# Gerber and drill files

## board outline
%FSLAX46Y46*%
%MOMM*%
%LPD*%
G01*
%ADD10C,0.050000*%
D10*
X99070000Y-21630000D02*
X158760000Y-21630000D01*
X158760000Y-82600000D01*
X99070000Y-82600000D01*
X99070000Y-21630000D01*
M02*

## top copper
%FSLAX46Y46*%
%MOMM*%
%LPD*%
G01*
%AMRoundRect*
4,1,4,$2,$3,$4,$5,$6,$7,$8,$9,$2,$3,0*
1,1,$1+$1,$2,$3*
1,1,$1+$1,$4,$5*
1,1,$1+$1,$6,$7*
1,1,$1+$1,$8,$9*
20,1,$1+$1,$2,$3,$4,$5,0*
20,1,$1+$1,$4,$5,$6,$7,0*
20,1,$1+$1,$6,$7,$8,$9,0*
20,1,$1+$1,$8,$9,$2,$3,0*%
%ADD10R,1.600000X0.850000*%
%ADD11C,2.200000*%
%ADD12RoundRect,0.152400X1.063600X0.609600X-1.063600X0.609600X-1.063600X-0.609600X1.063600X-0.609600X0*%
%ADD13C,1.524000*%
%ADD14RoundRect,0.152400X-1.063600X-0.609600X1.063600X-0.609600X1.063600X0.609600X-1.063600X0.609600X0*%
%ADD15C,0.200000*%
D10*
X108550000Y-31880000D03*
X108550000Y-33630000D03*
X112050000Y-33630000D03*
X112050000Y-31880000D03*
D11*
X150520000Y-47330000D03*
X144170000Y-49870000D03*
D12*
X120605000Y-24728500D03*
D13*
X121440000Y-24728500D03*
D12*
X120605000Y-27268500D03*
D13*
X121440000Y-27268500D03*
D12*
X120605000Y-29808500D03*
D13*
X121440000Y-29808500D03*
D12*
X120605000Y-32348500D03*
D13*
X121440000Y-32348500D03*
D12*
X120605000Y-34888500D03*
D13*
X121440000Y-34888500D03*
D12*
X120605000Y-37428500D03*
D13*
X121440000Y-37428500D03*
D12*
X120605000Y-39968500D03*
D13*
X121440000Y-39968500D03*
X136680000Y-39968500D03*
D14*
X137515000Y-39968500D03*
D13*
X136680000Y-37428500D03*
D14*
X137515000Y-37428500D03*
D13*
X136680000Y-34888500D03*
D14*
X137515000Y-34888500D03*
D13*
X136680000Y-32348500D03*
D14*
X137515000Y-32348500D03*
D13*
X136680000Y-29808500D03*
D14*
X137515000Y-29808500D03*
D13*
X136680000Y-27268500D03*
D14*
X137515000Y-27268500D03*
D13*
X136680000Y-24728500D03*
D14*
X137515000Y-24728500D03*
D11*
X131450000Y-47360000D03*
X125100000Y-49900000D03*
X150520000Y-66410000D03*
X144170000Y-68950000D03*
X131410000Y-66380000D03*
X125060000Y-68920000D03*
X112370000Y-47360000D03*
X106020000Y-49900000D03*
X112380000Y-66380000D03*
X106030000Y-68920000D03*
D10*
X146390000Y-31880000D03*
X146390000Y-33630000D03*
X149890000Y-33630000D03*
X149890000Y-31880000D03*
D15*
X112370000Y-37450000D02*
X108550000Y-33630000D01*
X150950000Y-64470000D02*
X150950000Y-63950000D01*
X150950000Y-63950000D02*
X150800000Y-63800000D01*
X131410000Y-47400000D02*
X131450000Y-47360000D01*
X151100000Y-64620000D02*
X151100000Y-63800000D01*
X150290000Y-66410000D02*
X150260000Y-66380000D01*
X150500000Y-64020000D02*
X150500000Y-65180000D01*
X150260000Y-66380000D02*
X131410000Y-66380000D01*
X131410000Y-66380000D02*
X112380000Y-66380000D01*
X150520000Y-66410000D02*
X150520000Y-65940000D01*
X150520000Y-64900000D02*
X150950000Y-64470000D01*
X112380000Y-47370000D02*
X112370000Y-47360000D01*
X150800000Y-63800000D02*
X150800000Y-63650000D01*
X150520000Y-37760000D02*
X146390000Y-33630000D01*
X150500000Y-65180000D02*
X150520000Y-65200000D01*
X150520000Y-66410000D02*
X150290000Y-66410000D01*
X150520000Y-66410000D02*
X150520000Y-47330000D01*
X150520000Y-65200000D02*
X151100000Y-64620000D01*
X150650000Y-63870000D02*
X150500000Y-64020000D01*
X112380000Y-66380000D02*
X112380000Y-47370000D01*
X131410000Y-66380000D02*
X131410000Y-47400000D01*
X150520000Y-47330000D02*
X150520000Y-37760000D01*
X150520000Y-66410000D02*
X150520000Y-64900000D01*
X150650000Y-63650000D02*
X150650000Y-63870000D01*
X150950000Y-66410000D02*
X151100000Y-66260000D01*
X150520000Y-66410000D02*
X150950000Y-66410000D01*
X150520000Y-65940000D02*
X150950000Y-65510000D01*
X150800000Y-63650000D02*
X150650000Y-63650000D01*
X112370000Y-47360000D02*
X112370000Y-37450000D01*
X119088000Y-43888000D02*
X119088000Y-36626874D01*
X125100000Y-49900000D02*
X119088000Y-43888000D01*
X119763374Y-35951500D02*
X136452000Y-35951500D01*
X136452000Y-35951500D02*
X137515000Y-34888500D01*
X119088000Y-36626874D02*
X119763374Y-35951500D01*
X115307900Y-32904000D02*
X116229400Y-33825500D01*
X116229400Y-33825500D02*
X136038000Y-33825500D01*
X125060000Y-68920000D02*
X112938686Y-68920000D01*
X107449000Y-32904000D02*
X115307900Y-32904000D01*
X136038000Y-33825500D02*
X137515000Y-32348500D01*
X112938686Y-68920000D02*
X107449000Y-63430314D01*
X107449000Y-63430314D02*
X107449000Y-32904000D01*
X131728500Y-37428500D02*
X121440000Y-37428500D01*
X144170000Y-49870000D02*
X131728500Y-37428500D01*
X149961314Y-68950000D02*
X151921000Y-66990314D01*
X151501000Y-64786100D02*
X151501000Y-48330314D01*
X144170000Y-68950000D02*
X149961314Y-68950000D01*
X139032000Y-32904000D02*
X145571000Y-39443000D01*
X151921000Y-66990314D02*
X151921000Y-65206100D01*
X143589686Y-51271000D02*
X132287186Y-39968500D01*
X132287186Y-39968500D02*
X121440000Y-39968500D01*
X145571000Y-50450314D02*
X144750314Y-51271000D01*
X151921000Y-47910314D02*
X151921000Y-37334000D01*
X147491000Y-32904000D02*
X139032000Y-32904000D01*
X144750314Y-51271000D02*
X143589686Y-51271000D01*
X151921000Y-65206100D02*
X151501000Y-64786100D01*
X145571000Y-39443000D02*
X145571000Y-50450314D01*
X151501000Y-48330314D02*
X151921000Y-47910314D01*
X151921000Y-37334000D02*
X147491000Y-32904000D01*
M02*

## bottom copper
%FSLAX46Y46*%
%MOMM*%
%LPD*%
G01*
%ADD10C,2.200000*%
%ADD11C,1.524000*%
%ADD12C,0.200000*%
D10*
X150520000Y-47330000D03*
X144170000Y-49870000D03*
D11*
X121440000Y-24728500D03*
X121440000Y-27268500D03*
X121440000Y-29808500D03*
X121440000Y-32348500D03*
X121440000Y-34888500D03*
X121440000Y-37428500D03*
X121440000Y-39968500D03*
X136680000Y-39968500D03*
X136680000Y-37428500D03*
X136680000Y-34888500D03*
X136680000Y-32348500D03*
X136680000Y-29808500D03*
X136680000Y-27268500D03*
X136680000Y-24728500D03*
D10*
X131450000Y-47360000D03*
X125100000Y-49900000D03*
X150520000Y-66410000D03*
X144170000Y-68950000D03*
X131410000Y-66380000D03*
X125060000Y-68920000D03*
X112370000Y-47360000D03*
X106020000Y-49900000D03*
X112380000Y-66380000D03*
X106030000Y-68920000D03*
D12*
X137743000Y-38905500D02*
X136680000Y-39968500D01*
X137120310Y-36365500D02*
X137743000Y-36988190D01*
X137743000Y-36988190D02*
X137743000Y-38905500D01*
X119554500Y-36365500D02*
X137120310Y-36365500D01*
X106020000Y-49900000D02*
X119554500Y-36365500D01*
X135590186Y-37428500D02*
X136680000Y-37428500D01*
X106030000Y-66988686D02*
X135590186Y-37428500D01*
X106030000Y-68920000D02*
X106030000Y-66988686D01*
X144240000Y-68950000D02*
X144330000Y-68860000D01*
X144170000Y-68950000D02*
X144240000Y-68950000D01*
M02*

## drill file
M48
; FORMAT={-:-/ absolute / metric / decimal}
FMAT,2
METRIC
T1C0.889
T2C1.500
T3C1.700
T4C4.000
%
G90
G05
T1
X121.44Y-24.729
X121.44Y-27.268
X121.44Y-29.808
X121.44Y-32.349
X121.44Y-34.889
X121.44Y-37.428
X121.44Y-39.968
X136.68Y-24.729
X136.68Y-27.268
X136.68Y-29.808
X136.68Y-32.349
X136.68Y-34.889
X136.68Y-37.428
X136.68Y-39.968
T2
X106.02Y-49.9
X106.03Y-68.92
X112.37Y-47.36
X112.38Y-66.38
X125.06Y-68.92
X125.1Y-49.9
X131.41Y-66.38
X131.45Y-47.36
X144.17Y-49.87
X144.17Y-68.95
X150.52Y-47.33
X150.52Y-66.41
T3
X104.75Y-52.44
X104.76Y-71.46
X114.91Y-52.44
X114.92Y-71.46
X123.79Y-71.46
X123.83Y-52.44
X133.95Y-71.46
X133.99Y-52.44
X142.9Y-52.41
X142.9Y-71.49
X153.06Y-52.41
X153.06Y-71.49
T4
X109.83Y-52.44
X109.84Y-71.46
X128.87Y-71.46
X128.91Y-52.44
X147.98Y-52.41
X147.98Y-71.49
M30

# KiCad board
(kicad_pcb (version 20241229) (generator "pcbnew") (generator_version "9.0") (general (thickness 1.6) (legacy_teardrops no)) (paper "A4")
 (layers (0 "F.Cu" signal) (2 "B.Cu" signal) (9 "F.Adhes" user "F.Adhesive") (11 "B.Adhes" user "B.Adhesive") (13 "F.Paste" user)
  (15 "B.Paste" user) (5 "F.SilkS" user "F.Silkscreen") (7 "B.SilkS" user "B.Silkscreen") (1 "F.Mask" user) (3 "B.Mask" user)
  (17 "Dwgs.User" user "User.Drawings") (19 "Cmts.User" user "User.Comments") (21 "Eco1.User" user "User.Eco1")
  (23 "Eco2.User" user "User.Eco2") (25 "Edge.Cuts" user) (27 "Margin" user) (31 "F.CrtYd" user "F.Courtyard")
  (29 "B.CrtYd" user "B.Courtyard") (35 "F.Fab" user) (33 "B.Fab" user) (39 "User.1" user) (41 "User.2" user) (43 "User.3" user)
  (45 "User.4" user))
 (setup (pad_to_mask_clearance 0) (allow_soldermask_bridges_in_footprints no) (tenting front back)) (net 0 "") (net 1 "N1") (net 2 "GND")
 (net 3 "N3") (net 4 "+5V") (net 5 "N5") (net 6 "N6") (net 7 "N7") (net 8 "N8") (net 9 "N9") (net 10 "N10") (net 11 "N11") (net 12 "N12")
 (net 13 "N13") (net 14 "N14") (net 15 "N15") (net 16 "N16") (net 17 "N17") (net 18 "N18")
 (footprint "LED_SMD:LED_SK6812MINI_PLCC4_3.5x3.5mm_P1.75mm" (layer "F.Cu") (at 110.3 32.755)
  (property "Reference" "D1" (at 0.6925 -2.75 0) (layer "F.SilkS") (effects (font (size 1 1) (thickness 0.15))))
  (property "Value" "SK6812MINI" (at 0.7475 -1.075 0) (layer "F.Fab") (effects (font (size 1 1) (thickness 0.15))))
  (pad "1" smd rect (at -1.75 -0.875) (size 1.6 0.85) (layers "F.Cu" "F.Mask" "F.Paste") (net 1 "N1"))
  (pad "2" smd rect (at -1.75 0.875) (size 1.6 0.85) (layers "F.Cu" "F.Mask" "F.Paste") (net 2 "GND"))
  (pad "3" smd rect (at 1.75 0.875) (size 1.6 0.85) (layers "F.Cu" "F.Mask" "F.Paste") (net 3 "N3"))
  (pad "4" smd rect (at 1.75 -0.875) (size 1.6 0.85) (layers "F.Cu" "F.Mask" "F.Paste") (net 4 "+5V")))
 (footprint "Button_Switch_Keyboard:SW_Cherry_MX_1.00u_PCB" (layer "F.Cu") (at 150.52 47.33)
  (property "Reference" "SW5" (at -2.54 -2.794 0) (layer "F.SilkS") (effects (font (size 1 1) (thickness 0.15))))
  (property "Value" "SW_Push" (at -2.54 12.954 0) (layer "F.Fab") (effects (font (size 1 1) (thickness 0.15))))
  (pad "" np_thru_hole circle (at -7.62 5.08) (size 1.7 1.7) (drill 1.7) (layers "*.Cu" "*.Mask"))
  (pad "" np_thru_hole circle (at -2.54 5.08) (size 4 4) (drill 4) (layers "*.Cu" "*.Mask"))
  (pad "" np_thru_hole circle (at 2.54 5.08) (size 1.7 1.7) (drill 1.7) (layers "*.Cu" "*.Mask"))
  (pad "1" thru_hole circle (at 0 0) (size 2.2 2.2) (drill 1.5) (layers "*.Cu" "*.Mask") (remove_unused_layers no) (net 2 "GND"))
  (pad "2" thru_hole circle (at -6.35 2.54) (size 2.2 2.2) (drill 1.5) (layers "*.Cu" "*.Mask") (remove_unused_layers no) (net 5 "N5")))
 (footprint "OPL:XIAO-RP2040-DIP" (layer "F.Cu") (at 129.06 32.3485)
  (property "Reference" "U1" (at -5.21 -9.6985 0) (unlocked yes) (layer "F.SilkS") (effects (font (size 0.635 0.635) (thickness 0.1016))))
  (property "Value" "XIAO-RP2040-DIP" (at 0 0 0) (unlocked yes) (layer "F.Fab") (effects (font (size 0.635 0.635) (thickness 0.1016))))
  (pad "1" smd roundrect (at -8.455 -7.62 180) (size 2.432 1.524) (layers "F.Cu" "F.Mask") (roundrect_rratio 0.1) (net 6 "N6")
   (thermal_bridge_angle 45))
  (pad "1" thru_hole circle (at -7.62 -7.62 180) (size 1.524 1.524) (drill 0.889) (layers "*.Cu" "*.Mask") (remove_unused_layers no)
   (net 6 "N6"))
  (pad "2" smd roundrect (at -8.455 -5.08 180) (size 2.432 1.524) (layers "F.Cu" "F.Mask") (roundrect_rratio 0.1) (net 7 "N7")
   (thermal_bridge_angle 45))
  (pad "2" thru_hole circle (at -7.62 -5.08 180) (size 1.524 1.524) (drill 0.889) (layers "*.Cu" "*.Mask") (remove_unused_layers no)
   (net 7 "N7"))
  (pad "3" smd roundrect (at -8.455 -2.54 180) (size 2.432 1.524) (layers "F.Cu" "F.Mask") (roundrect_rratio 0.1) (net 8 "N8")
   (thermal_bridge_angle 45))
  (pad "3" thru_hole circle (at -7.62 -2.54 180) (size 1.524 1.524) (drill 0.889) (layers "*.Cu" "*.Mask") (remove_unused_layers no)
   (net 8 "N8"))
  (pad "4" smd roundrect (at -8.455 0 180) (size 2.432 1.524) (layers "F.Cu" "F.Mask") (roundrect_rratio 0.1) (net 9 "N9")
   (thermal_bridge_angle 45))
  (pad "4" thru_hole circle (at -7.62 0 180) (size 1.524 1.524) (drill 0.889) (layers "*.Cu" "*.Mask") (remove_unused_layers no)
   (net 9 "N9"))
  (pad "5" smd roundrect (at -8.455 2.54 180) (size 2.432 1.524) (layers "F.Cu" "F.Mask") (roundrect_rratio 0.1) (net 3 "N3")
   (thermal_bridge_angle 45))
  (pad "5" thru_hole circle (at -7.62 2.54 180) (size 1.524 1.524) (drill 0.889) (layers "*.Cu" "*.Mask") (remove_unused_layers no)
   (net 3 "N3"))
  (pad "6" smd roundrect (at -8.455 5.08 180) (size 2.432 1.524) (layers "F.Cu" "F.Mask") (roundrect_rratio 0.1) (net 5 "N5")
   (thermal_bridge_angle 45))
  (pad "6" thru_hole circle (at -7.62 5.08 180) (size 1.524 1.524) (drill 0.889) (layers "*.Cu" "*.Mask") (remove_unused_layers no)
   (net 5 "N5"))
  (pad "7" smd roundrect (at -8.455 7.62 180) (size 2.432 1.524) (layers "F.Cu" "F.Mask") (roundrect_rratio 0.1) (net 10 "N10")
   (thermal_bridge_angle 45))
  (pad "7" thru_hole circle (at -7.62 7.62 180) (size 1.524 1.524) (drill 0.889) (layers "*.Cu" "*.Mask") (remove_unused_layers no)
   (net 10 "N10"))
  (pad "8" thru_hole circle (at 7.62 7.62) (size 1.524 1.524) (drill 0.889) (layers "*.Cu" "*.Mask") (remove_unused_layers no)
   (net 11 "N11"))
  (pad "8" smd roundrect (at 8.455 7.62) (size 2.432 1.524) (layers "F.Cu" "F.Mask") (roundrect_rratio 0.1) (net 11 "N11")
   (thermal_bridge_angle 45))
  (pad "9" thru_hole circle (at 7.62 5.08) (size 1.524 1.524) (drill 0.889) (layers "*.Cu" "*.Mask") (remove_unused_layers no)
   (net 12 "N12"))
  (pad "9" smd roundrect (at 8.455 5.08) (size 2.432 1.524) (layers "F.Cu" "F.Mask") (roundrect_rratio 0.1) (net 12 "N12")
   (thermal_bridge_angle 45))
  (pad "10" thru_hole circle (at 7.62 2.54) (size 1.524 1.524) (drill 0.889) (layers "*.Cu" "*.Mask") (remove_unused_layers no)
   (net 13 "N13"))
  (pad "10" smd roundrect (at 8.455 2.54) (size 2.432 1.524) (layers "F.Cu" "F.Mask") (roundrect_rratio 0.1) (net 13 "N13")
   (thermal_bridge_angle 45))
  (pad "11" thru_hole circle (at 7.62 0) (size 1.524 1.524) (drill 0.889) (layers "*.Cu" "*.Mask") (remove_unused_layers no) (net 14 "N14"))
  (pad "11" smd roundrect (at 8.455 0) (size 2.432 1.524) (layers "F.Cu" "F.Mask") (roundrect_rratio 0.1) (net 14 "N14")
   (thermal_bridge_angle 45))
  (pad "12" thru_hole circle (at 7.62 -2.54) (size 1.524 1.524) (drill 0.889) (layers "*.Cu" "*.Mask") (remove_unused_layers no)
   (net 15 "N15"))
  (pad "12" smd roundrect (at 8.455 -2.54) (size 2.432 1.524) (layers "F.Cu" "F.Mask") (roundrect_rratio 0.1) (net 15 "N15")
   (thermal_bridge_angle 45))
  (pad "13" thru_hole circle (at 7.62 -5.08) (size 1.524 1.524) (drill 0.889) (layers "*.Cu" "*.Mask") (remove_unused_layers no)
   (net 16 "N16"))
  (pad "13" smd roundrect (at 8.455 -5.08) (size 2.432 1.524) (layers "F.Cu" "F.Mask") (roundrect_rratio 0.1) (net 16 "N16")
   (thermal_bridge_angle 45))
  (pad "14" thru_hole circle (at 7.62 -7.62) (size 1.524 1.524) (drill 0.889) (layers "*.Cu" "*.Mask") (remove_unused_layers no)
   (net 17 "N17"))
  (pad "14" smd roundrect (at 8.455 -7.62) (size 2.432 1.524) (layers "F.Cu" "F.Mask") (roundrect_rratio 0.1) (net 17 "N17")
   (thermal_bridge_angle 45)))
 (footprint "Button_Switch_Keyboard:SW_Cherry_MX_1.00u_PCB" (layer "F.Cu") (at 131.45 47.36)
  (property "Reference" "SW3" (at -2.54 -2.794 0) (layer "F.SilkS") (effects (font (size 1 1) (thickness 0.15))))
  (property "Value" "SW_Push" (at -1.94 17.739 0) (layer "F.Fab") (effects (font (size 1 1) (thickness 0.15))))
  (pad "" np_thru_hole circle (at -7.62 5.08) (size 1.7 1.7) (drill 1.7) (layers "*.Cu" "*.Mask"))
  (pad "" np_thru_hole circle (at -2.54 5.08) (size 4 4) (drill 4) (layers "*.Cu" "*.Mask"))
  (pad "" np_thru_hole circle (at 2.54 5.08) (size 1.7 1.7) (drill 1.7) (layers "*.Cu" "*.Mask"))
  (pad "1" thru_hole circle (at 0 0) (size 2.2 2.2) (drill 1.5) (layers "*.Cu" "*.Mask") (remove_unused_layers no) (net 2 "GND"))
  (pad "2" thru_hole circle (at -6.35 2.54) (size 2.2 2.2) (drill 1.5) (layers "*.Cu" "*.Mask") (remove_unused_layers no) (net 13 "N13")))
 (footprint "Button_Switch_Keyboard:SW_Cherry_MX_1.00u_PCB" (layer "F.Cu") (at 150.52 66.41)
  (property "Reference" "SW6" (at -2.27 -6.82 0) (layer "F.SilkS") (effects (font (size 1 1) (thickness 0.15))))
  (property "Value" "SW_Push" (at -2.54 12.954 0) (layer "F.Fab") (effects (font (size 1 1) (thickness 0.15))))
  (pad "" np_thru_hole circle (at -7.62 5.08) (size 1.7 1.7) (drill 1.7) (layers "*.Cu" "*.Mask"))
  (pad "" np_thru_hole circle (at -2.54 5.08) (size 4 4) (drill 4) (layers "*.Cu" "*.Mask"))
  (pad "" np_thru_hole circle (at 2.54 5.08) (size 1.7 1.7) (drill 1.7) (layers "*.Cu" "*.Mask"))
  (pad "1" thru_hole circle (at 0 0) (size 2.2 2.2) (drill 1.5) (layers "*.Cu" "*.Mask") (remove_unused_layers no) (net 2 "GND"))
  (pad "2" thru_hole circle (at -6.35 2.54) (size 2.2 2.2) (drill 1.5) (layers "*.Cu" "*.Mask") (remove_unused_layers no) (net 10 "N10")))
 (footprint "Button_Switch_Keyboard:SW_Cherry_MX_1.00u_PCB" (layer "F.Cu") (at 131.41 66.38)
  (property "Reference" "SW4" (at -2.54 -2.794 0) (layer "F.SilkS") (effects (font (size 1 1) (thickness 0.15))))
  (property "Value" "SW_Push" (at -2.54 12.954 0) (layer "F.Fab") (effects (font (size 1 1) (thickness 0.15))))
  (pad "" np_thru_hole circle (at -7.62 5.08) (size 1.7 1.7) (drill 1.7) (layers "*.Cu" "*.Mask"))
  (pad "" np_thru_hole circle (at -2.54 5.08) (size 4 4) (drill 4) (layers "*.Cu" "*.Mask"))
  (pad "" np_thru_hole circle (at 2.54 5.08) (size 1.7 1.7) (drill 1.7) (layers "*.Cu" "*.Mask"))
  (pad "1" thru_hole circle (at 0 0) (size 2.2 2.2) (drill 1.5) (layers "*.Cu" "*.Mask") (remove_unused_layers no) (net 2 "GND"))
  (pad "2" thru_hole circle (at -6.35 2.54) (size 2.2 2.2) (drill 1.5) (layers "*.Cu" "*.Mask") (remove_unused_layers no) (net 14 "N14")))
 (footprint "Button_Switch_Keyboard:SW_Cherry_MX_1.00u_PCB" (layer "F.Cu") (at 112.37 47.36)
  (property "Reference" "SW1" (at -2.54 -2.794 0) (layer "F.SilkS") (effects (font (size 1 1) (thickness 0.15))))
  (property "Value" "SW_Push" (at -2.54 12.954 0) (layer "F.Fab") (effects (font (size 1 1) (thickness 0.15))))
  (pad "" np_thru_hole circle (at -7.62 5.08) (size 1.7 1.7) (drill 1.7) (layers "*.Cu" "*.Mask"))
  (pad "" np_thru_hole circle (at -2.54 5.08) (size 4 4) (drill 4) (layers "*.Cu" "*.Mask"))
  (pad "" np_thru_hole circle (at 2.54 5.08) (size 1.7 1.7) (drill 1.7) (layers "*.Cu" "*.Mask"))
  (pad "1" thru_hole circle (at 0 0) (size 2.2 2.2) (drill 1.5) (layers "*.Cu" "*.Mask") (remove_unused_layers no) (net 2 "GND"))
  (pad "2" thru_hole circle (at -6.35 2.54) (size 2.2 2.2) (drill 1.5) (layers "*.Cu" "*.Mask") (remove_unused_layers no) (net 11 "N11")))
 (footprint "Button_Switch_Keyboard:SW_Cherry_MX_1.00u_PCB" (layer "F.Cu") (at 112.38 66.38)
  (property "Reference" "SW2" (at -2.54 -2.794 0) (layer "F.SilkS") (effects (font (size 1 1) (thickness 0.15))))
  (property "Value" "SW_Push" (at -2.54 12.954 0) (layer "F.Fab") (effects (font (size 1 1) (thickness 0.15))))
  (pad "" np_thru_hole circle (at -7.62 5.08) (size 1.7 1.7) (drill 1.7) (layers "*.Cu" "*.Mask"))
  (pad "" np_thru_hole circle (at -2.54 5.08) (size 4 4) (drill 4) (layers "*.Cu" "*.Mask"))
  (pad "" np_thru_hole circle (at 2.54 5.08) (size 1.7 1.7) (drill 1.7) (layers "*.Cu" "*.Mask"))
  (pad "1" thru_hole circle (at 0 0) (size 2.2 2.2) (drill 1.5) (layers "*.Cu" "*.Mask") (remove_unused_layers no) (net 2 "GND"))
  (pad "2" thru_hole circle (at -6.35 2.54) (size 2.2 2.2) (drill 1.5) (layers "*.Cu" "*.Mask") (remove_unused_layers no) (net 12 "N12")))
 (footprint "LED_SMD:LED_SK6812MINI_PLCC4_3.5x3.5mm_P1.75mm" (layer "F.Cu") (at 148.14 32.755)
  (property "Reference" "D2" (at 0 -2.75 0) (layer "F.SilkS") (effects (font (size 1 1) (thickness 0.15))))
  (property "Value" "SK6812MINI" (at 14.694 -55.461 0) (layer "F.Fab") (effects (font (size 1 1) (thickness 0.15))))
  (pad "1" smd rect (at -1.75 -0.875) (size 1.6 0.85) (layers "F.Cu" "F.Mask" "F.Paste") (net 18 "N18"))
  (pad "2" smd rect (at -1.75 0.875) (size 1.6 0.85) (layers "F.Cu" "F.Mask" "F.Paste") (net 2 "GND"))
  (pad "3" smd rect (at 1.75 0.875) (size 1.6 0.85) (layers "F.Cu" "F.Mask" "F.Paste") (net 1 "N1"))
  (pad "4" smd rect (at 1.75 -0.875) (size 1.6 0.85) (layers "F.Cu" "F.Mask" "F.Paste") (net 4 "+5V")))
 (gr_rect (start 99.07 21.63) (end 158.76 82.6) (stroke (width 0.05) (type default)) (fill no) (layer "Edge.Cuts"))
 (segment (start 112.37 37.45) (end 108.55 33.63) (width 0.2) (layer "F.Cu") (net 2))
 (segment (start 150.95 64.47) (end 150.95 63.95) (width 0.2) (layer "F.Cu") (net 2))
 (segment (start 150.95 63.95) (end 150.8 63.8) (width 0.2) (layer "F.Cu") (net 2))
 (segment (start 131.41 47.4) (end 131.45 47.36) (width 0.2) (layer "F.Cu") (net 2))
 (segment (start 151.1 64.62) (end 151.1 63.8) (width 0.2) (layer "F.Cu") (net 2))
 (segment (start 150.29 66.41) (end 150.26 66.38) (width 0.2) (layer "F.Cu") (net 2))
 (segment (start 150.5 64.02) (end 150.5 65.18) (width 0.2) (layer "F.Cu") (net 2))
 (segment (start 150.26 66.38) (end 131.41 66.38) (width 0.2) (layer "F.Cu") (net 2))
 (segment (start 131.41 66.38) (end 112.38 66.38) (width 0.2) (layer "F.Cu") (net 2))
 (segment (start 150.52 66.41) (end 150.52 65.94) (width 0.2) (layer "F.Cu") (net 2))
 (segment (start 150.52 64.9) (end 150.95 64.47) (width 0.2) (layer "F.Cu") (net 2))
 (segment (start 112.38 47.37) (end 112.37 47.36) (width 0.2) (layer "F.Cu") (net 2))
 (segment (start 150.8 63.8) (end 150.8 63.65) (width 0.2) (layer "F.Cu") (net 2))
 (segment (start 150.52 37.76) (end 146.39 33.63) (width 0.2) (layer "F.Cu") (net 2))
 (segment (start 150.5 65.18) (end 150.52 65.2) (width 0.2) (layer "F.Cu") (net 2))
 (segment (start 150.52 66.41) (end 150.29 66.41) (width 0.2) (layer "F.Cu") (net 2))
 (segment (start 150.52 66.41) (end 150.52 47.33) (width 0.2) (layer "F.Cu") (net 2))
 (segment (start 150.52 65.2) (end 151.1 64.62) (width 0.2) (layer "F.Cu") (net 2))
 (segment (start 150.65 63.87) (end 150.5 64.02) (width 0.2) (layer "F.Cu") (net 2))
 (segment (start 112.38 66.38) (end 112.38 47.37) (width 0.2) (layer "F.Cu") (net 2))
 (segment (start 131.41 66.38) (end 131.41 47.4) (width 0.2) (layer "F.Cu") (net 2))
 (segment (start 150.52 47.33) (end 150.52 37.76) (width 0.2) (layer "F.Cu") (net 2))
 (segment (start 150.52 66.41) (end 150.52 64.9) (width 0.2) (layer "F.Cu") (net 2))
 (segment (start 150.65 63.65) (end 150.65 63.87) (width 0.2) (layer "F.Cu") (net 2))
 (segment (start 150.95 66.41) (end 151.1 66.26) (width 0.2) (layer "F.Cu") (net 2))
 (segment (start 150.52 66.41) (end 150.95 66.41) (width 0.2) (layer "F.Cu") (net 2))
 (segment (start 150.52 65.94) (end 150.95 65.51) (width 0.2) (layer "F.Cu") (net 2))
 (segment (start 150.8 63.65) (end 150.65 63.65) (width 0.2) (layer "F.Cu") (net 2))
 (segment (start 112.37 47.36) (end 112.37 37.45) (width 0.2) (layer "F.Cu") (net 2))
 (segment (start 137.743 38.9055) (end 136.68 39.9685) (width 0.2) (layer "B.Cu") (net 11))
 (segment (start 137.12031 36.3655) (end 137.743 36.98819) (width 0.2) (layer "B.Cu") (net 11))
 (segment (start 137.743 36.98819) (end 137.743 38.9055) (width 0.2) (layer "B.Cu") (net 11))
 (segment (start 119.5545 36.3655) (end 137.12031 36.3655) (width 0.2) (layer "B.Cu") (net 11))
 (segment (start 106.02 49.9) (end 119.5545 36.3655) (width 0.2) (layer "B.Cu") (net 11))
 (segment (start 135.590186 37.4285) (end 136.68 37.4285) (width 0.2) (layer "B.Cu") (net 12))
 (segment (start 106.03 66.988686) (end 135.590186 37.4285) (width 0.2) (layer "B.Cu") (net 12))
 (segment (start 106.03 68.92) (end 106.03 66.988686) (width 0.2) (layer "B.Cu") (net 12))
 (segment (start 119.088 43.888) (end 119.088 36.626874) (width 0.2) (layer "F.Cu") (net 13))
 (segment (start 125.1 49.9) (end 119.088 43.888) (width 0.2) (layer "F.Cu") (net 13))
 (segment (start 119.763374 35.9515) (end 136.452 35.9515) (width 0.2) (layer "F.Cu") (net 13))
 (segment (start 136.452 35.9515) (end 137.515 34.8885) (width 0.2) (layer "F.Cu") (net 13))
 (segment (start 119.088 36.626874) (end 119.763374 35.9515) (width 0.2) (layer "F.Cu") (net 13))
 (segment (start 115.3079 32.904) (end 116.2294 33.8255) (width 0.2) (layer "F.Cu") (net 14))
 (segment (start 116.2294 33.8255) (end 136.038 33.8255) (width 0.2) (layer "F.Cu") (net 14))
 (segment (start 125.06 68.92) (end 112.938686 68.92) (width 0.2) (layer "F.Cu") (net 14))
 (segment (start 107.449 32.904) (end 115.3079 32.904) (width 0.2) (layer "F.Cu") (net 14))
 (segment (start 136.038 33.8255) (end 137.515 32.3485) (width 0.2) (layer "F.Cu") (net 14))
 (segment (start 112.938686 68.92) (end 107.449 63.430314) (width 0.2) (layer "F.Cu") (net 14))
 (segment (start 107.449 63.430314) (end 107.449 32.904) (width 0.2) (layer "F.Cu") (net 14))
 (segment (start 131.7285 37.4285) (end 121.44 37.4285) (width 0.2) (layer "F.Cu") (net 5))
 (segment (start 144.17 49.87) (end 131.7285 37.4285) (width 0.2) (layer "F.Cu") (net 5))
 (segment (start 149.961314 68.95) (end 151.921 66.990314) (width 0.2) (layer "F.Cu") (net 10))
 (segment (start 151.501 64.7861) (end 151.501 48.330314) (width 0.2) (layer "F.Cu") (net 10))
 (segment (start 144.17 68.95) (end 149.961314 68.95) (width 0.2) (layer "F.Cu") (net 10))
 (segment (start 139.032 32.904) (end 145.571 39.443) (width 0.2) (layer "F.Cu") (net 10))
 (segment (start 151.921 66.990314) (end 151.921 65.2061) (width 0.2) (layer "F.Cu") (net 10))
 (segment (start 143.589686 51.271) (end 132.287186 39.9685) (width 0.2) (layer "F.Cu") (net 10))
 (segment (start 132.287186 39.9685) (end 121.44 39.9685) (width 0.2) (layer "F.Cu") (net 10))
 (segment (start 145.571 50.450314) (end 144.750314 51.271) (width 0.2) (layer "F.Cu") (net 10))
 (segment (start 151.921 47.910314) (end 151.921 37.334) (width 0.2) (layer "F.Cu") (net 10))
 (segment (start 147.491 32.904) (end 139.032 32.904) (width 0.2) (layer "F.Cu") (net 10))
 (segment (start 144.750314 51.271) (end 143.589686 51.271) (width 0.2) (layer "F.Cu") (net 10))
 (segment (start 151.921 65.2061) (end 151.501 64.7861) (width 0.2) (layer "F.Cu") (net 10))
 (segment (start 145.571 39.443) (end 145.571 50.450314) (width 0.2) (layer "F.Cu") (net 10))
 (segment (start 151.501 48.330314) (end 151.921 47.910314) (width 0.2) (layer "F.Cu") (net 10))
 (segment (start 151.921 37.334) (end 147.491 32.904) (width 0.2) (layer "F.Cu") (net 10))
 (segment (start 144.24 68.95) (end 144.33 68.86) (width 0.2) (layer "B.Cu") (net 10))
 (segment (start 144.17 68.95) (end 144.24 68.95) (width 0.2) (layer "B.Cu") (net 10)))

